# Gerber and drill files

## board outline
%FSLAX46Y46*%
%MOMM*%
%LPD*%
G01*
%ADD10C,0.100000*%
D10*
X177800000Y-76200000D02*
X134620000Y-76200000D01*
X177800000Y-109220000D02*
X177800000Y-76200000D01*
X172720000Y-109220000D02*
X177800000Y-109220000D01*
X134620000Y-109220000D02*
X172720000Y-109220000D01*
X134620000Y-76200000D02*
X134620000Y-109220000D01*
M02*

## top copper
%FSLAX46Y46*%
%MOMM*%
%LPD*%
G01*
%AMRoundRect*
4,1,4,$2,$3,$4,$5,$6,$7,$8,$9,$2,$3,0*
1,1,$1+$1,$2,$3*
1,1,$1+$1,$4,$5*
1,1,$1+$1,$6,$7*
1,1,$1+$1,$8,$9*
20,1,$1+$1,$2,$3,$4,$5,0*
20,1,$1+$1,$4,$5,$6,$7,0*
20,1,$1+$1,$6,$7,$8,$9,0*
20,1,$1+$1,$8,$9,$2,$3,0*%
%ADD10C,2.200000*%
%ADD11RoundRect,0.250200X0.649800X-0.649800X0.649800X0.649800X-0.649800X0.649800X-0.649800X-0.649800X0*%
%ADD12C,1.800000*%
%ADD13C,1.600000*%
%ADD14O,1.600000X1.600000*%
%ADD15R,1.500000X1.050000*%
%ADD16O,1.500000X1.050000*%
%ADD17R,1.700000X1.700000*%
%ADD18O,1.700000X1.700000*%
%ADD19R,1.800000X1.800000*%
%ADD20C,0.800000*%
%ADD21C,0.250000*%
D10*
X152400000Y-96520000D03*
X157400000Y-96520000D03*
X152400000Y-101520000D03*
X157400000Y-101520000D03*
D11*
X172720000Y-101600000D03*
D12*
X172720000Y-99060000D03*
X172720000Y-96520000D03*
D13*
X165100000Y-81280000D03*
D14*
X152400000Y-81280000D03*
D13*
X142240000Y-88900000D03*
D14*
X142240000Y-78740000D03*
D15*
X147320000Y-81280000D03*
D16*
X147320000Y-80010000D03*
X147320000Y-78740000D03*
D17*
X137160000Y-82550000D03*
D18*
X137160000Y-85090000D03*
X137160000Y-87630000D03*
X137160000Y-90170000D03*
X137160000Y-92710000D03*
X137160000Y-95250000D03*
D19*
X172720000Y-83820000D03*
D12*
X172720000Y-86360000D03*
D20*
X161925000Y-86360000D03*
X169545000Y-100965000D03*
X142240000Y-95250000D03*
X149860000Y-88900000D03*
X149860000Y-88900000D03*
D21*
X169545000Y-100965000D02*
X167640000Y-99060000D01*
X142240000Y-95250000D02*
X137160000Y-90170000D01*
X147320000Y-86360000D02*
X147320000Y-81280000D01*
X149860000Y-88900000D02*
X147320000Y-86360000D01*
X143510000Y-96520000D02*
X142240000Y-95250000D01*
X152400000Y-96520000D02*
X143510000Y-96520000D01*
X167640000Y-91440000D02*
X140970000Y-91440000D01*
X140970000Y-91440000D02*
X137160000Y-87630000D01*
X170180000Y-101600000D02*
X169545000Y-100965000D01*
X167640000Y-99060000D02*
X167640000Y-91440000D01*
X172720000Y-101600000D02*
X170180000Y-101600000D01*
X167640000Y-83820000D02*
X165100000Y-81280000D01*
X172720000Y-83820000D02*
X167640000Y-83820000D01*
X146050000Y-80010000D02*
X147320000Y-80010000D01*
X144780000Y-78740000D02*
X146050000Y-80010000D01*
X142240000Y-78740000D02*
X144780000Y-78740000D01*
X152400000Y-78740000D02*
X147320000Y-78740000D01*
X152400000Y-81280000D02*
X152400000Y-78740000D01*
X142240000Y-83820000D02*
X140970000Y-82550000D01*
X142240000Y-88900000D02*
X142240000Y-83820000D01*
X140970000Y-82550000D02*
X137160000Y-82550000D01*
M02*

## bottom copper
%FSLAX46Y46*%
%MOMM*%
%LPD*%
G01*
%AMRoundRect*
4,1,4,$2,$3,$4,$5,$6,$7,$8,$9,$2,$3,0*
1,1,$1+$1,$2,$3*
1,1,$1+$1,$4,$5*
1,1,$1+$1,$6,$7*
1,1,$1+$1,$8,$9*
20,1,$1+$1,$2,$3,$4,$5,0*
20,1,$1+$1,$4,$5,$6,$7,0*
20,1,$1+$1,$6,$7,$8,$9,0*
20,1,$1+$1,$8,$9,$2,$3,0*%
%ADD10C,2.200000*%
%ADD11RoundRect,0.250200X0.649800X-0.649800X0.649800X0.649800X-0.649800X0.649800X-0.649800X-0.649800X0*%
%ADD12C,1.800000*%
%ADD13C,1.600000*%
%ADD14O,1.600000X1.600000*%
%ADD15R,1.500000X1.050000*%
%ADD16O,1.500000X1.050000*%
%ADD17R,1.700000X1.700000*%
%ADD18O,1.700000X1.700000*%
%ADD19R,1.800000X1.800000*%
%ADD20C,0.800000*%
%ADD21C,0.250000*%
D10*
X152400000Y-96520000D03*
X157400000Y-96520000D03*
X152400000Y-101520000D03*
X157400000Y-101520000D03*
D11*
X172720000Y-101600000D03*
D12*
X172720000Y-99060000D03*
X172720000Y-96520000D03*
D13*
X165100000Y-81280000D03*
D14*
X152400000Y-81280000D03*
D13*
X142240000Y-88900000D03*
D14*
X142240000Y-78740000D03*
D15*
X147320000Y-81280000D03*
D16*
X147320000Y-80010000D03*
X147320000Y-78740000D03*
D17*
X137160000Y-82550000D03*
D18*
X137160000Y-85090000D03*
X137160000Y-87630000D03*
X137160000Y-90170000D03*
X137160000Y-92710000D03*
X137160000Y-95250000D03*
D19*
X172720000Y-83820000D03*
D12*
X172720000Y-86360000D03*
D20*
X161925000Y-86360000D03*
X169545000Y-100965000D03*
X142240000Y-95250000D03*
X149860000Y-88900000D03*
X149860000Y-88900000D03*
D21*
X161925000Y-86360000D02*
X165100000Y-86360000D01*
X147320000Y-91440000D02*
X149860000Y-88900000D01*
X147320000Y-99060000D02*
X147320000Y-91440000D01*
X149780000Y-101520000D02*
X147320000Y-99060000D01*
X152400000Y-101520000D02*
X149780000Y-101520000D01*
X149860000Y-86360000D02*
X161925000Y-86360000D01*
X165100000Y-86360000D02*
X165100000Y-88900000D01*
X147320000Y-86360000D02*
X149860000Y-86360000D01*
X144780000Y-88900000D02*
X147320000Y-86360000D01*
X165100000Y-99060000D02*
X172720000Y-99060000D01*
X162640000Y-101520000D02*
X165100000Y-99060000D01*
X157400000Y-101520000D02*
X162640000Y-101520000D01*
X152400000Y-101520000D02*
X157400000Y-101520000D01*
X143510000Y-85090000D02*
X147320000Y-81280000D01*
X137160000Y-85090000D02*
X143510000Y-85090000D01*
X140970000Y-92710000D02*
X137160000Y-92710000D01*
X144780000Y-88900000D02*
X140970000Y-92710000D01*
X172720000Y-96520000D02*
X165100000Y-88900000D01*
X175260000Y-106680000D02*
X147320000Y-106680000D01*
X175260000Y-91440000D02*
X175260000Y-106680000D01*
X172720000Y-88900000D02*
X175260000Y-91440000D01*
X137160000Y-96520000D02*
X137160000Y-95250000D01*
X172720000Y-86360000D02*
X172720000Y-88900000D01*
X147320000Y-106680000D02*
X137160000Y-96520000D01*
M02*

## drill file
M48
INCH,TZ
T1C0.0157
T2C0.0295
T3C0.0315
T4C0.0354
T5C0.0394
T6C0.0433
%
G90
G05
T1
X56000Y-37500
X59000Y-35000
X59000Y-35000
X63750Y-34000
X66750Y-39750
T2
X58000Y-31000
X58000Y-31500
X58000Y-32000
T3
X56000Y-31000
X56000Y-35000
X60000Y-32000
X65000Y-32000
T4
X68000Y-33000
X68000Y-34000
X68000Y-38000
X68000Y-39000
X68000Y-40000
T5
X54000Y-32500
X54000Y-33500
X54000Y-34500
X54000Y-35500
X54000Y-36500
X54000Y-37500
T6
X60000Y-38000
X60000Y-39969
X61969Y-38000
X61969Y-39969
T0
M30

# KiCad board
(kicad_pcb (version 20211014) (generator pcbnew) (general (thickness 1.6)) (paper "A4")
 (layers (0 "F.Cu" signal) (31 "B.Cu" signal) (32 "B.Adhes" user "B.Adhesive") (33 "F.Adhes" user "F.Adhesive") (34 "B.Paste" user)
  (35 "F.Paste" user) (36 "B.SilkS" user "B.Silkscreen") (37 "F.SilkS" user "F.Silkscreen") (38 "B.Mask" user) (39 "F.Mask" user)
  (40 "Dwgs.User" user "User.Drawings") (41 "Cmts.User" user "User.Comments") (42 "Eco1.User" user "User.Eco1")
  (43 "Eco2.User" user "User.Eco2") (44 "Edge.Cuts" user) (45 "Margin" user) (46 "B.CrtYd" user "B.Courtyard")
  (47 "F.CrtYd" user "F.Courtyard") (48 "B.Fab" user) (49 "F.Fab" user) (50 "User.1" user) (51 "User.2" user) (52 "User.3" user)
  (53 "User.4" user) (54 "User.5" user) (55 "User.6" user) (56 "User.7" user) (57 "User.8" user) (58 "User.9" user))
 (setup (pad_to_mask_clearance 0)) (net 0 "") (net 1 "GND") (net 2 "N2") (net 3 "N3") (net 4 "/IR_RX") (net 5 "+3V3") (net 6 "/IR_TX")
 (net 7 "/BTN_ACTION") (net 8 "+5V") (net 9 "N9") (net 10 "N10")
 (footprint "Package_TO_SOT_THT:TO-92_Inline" (layer "F.Cu") (at 147.32 81.28 90)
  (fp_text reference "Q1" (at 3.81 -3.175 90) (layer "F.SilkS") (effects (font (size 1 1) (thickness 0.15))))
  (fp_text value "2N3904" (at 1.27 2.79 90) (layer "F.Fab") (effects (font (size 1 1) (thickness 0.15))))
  (pad "1" thru_hole rect (at 0 0 90) (size 1.05 1.5) (drill 0.75) (layers *.Cu *.Mask) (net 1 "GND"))
  (pad "2" thru_hole oval (at 1.27 0 90) (size 1.05 1.5) (drill 0.75) (layers *.Cu *.Mask) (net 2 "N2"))
  (pad "3" thru_hole oval (at 2.54 0 90) (size 1.05 1.5) (drill 0.75) (layers *.Cu *.Mask) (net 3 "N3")))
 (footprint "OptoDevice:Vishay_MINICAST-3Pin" (layer "F.Cu") (at 172.72 101.6 90)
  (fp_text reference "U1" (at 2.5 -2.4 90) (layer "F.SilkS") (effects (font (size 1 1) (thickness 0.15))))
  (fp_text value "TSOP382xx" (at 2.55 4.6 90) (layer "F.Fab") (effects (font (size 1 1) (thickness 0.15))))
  (pad "1" thru_hole roundrect (at 0 0 90) (size 1.8 1.8) (drill 0.9) (layers *.Cu *.Mask) (roundrect_rratio 0.139) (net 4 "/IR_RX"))
  (pad "2" thru_hole circle (at 2.54 0 90) (size 1.8 1.8) (drill 0.9) (layers *.Cu *.Mask) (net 1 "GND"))
  (pad "3" thru_hole circle (at 5.08 0 90) (size 1.8 1.8) (drill 0.9) (layers *.Cu *.Mask) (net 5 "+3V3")))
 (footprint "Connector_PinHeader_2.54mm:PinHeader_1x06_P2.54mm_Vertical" (layer "F.Cu") (at 137.16 82.55)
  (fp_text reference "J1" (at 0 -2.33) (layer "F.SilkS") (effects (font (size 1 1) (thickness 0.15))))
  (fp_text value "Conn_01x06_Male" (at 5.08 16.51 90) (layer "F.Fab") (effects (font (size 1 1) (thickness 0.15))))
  (pad "1" thru_hole rect (at 0 0) (size 1.7 1.7) (drill 1) (layers *.Cu *.Mask) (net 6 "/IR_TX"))
  (pad "2" thru_hole oval (at 0 2.54) (size 1.7 1.7) (drill 1) (layers *.Cu *.Mask) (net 1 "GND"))
  (pad "3" thru_hole oval (at 0 5.08) (size 1.7 1.7) (drill 1) (layers *.Cu *.Mask) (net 4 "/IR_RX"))
  (pad "4" thru_hole oval (at 0 7.62) (size 1.7 1.7) (drill 1) (layers *.Cu *.Mask) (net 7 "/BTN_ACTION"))
  (pad "5" thru_hole oval (at 0 10.16) (size 1.7 1.7) (drill 1) (layers *.Cu *.Mask) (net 5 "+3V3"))
  (pad "6" thru_hole oval (at 0 12.7) (size 1.7 1.7) (drill 1) (layers *.Cu *.Mask) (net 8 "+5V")))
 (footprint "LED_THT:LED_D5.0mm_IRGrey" (layer "F.Cu") (at 172.72 83.82 -90)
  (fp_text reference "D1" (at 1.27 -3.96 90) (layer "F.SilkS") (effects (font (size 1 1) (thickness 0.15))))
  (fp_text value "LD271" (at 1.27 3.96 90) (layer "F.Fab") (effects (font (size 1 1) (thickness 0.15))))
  (pad "1" thru_hole rect (at 0 0 270) (size 1.8 1.8) (drill 0.9) (layers *.Cu *.Mask) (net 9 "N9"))
  (pad "2" thru_hole circle (at 2.54 0 270) (size 1.8 1.8) (drill 0.9) (layers *.Cu *.Mask) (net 8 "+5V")))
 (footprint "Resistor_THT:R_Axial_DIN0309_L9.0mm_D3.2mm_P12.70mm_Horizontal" (layer "F.Cu") (at 165.1 81.28 180)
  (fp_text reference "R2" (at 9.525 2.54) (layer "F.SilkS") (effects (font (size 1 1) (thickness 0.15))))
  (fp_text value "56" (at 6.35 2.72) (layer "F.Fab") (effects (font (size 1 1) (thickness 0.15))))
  (pad "1" thru_hole circle (at 0 0 180) (size 1.6 1.6) (drill 0.8) (layers *.Cu *.Mask) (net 9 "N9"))
  (pad "2" thru_hole oval (at 12.7 0 180) (size 1.6 1.6) (drill 0.8) (layers *.Cu *.Mask) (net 3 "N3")))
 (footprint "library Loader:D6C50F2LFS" (layer "F.Cu") (at 152.4 96.52)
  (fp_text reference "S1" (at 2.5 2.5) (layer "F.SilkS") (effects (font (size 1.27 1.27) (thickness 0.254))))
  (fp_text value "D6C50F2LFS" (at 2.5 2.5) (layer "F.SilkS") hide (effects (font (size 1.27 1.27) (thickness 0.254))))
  (pad "1" thru_hole circle locked (at 0 0) (size 2.2 2.2) (drill 1.1) (layers *.Cu *.Mask) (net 7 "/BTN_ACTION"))
  (pad "2" thru_hole circle locked (at 5 0) (size 2.2 2.2) (drill 1.1) (layers *.Cu *.Mask) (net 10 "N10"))
  (pad "3" thru_hole circle locked (at 0 5) (size 2.2 2.2) (drill 1.1) (layers *.Cu *.Mask) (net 1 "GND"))
  (pad "4" thru_hole circle locked (at 5 5) (size 2.2 2.2) (drill 1.1) (layers *.Cu *.Mask) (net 1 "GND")))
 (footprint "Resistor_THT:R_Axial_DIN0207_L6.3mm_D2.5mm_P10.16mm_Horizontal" (layer "F.Cu") (at 142.24 88.9 90)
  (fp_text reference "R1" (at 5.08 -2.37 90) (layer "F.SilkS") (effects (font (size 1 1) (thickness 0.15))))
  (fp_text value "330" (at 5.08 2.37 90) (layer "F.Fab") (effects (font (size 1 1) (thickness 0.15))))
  (pad "1" thru_hole circle (at 0 0 90) (size 1.6 1.6) (drill 0.8) (layers *.Cu *.Mask) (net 6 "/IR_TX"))
  (pad "2" thru_hole oval (at 10.16 0 90) (size 1.6 1.6) (drill 0.8) (layers *.Cu *.Mask) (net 2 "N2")))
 (gr_line (start 177.8 76.2) (end 134.62 76.2) (layer "Edge.Cuts") (width 0.1))
 (gr_line (start 134.62 109.22) (end 172.72 109.22) (layer "Edge.Cuts") (width 0.1))
 (gr_line (start 172.72 109.22) (end 177.8 109.22) (layer "Edge.Cuts") (width 0.1))
 (gr_line (start 177.8 109.22) (end 177.8 76.2) (layer "Edge.Cuts") (width 0.1))
 (gr_line (start 134.62 76.2) (end 134.62 109.22) (layer "Edge.Cuts") (width 0.1))
 (segment (start 172.72 83.82) (end 167.64 83.82) (width 0.25) (layer "F.Cu") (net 9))
 (segment (start 167.64 83.82) (end 165.1 81.28) (width 0.25) (layer "F.Cu") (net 9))
 (segment (start 147.32 106.68) (end 137.16 96.52) (width 0.25) (layer "B.Cu") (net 8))
 (segment (start 172.72 88.9) (end 175.26 91.44) (width 0.25) (layer "B.Cu") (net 8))
 (segment (start 175.26 91.44) (end 175.26 106.68) (width 0.25) (layer "B.Cu") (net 8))
 (segment (start 175.26 106.68) (end 147.32 106.68) (width 0.25) (layer "B.Cu") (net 8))
 (segment (start 137.16 96.52) (end 137.16 95.25) (width 0.25) (layer "B.Cu") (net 8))
 (segment (start 172.72 86.36) (end 172.72 88.9) (width 0.25) (layer "B.Cu") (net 8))
 (segment (start 142.24 88.9) (end 142.24 83.82) (width 0.25) (layer "F.Cu") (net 6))
 (segment (start 140.97 82.55) (end 137.16 82.55) (width 0.25) (layer "F.Cu") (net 6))
 (segment (start 142.24 83.82) (end 140.97 82.55) (width 0.25) (layer "F.Cu") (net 6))
 (segment (start 147.32 86.36) (end 147.32 81.28) (width 0.25) (layer "F.Cu") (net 1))
 (segment (start 149.86 88.9) (end 147.32 86.36) (width 0.25) (layer "F.Cu") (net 1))
 (via (at 149.86 88.9) (size 0.8) (drill 0.4) (layers "F.Cu" "B.Cu") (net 1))
 (via (at 149.86 88.9) (size 0.8) (drill 0.4) (layers "F.Cu" "B.Cu") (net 1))
 (segment (start 137.16 85.09) (end 143.51 85.09) (width 0.25) (layer "B.Cu") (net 1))
 (segment (start 152.4 101.52) (end 149.78 101.52) (width 0.25) (layer "B.Cu") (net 1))
 (segment (start 152.4 101.52) (end 157.4 101.52) (width 0.25) (layer "B.Cu") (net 1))
 (segment (start 143.51 85.09) (end 147.32 81.28) (width 0.25) (layer "B.Cu") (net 1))
 (segment (start 162.64 101.52) (end 165.1 99.06) (width 0.25) (layer "B.Cu") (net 1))
 (segment (start 157.4 101.52) (end 162.64 101.52) (width 0.25) (layer "B.Cu") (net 1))
 (segment (start 147.32 91.44) (end 149.86 88.9) (width 0.25) (layer "B.Cu") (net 1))
 (segment (start 149.78 101.52) (end 147.32 99.06) (width 0.25) (layer "B.Cu") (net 1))
 (segment (start 147.32 99.06) (end 147.32 91.44) (width 0.25) (layer "B.Cu") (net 1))
 (segment (start 165.1 99.06) (end 172.72 99.06) (width 0.25) (layer "B.Cu") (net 1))
 (segment (start 172.72 101.6) (end 170.18 101.6) (width 0.25) (layer "F.Cu") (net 4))
 (segment (start 170.18 101.6) (end 169.545 100.965) (width 0.25) (layer "F.Cu") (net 4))
 (segment (start 140.97 91.44) (end 137.16 87.63) (width 0.25) (layer "F.Cu") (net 4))
 (segment (start 167.64 91.44) (end 140.97 91.44) (width 0.25) (layer "F.Cu") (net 4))
 (segment (start 167.64 99.06) (end 167.64 91.44) (width 0.25) (layer "F.Cu") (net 4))
 (segment (start 169.545 100.965) (end 167.64 99.06) (width 0.25) (layer "F.Cu") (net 4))
 (via (at 169.545 100.965) (size 0.8) (drill 0.4) (layers "F.Cu" "B.Cu") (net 4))
 (segment (start 152.4 96.52) (end 143.51 96.52) (width 0.25) (layer "F.Cu") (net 7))
 (segment (start 142.24 95.25) (end 137.16 90.17) (width 0.25) (layer "F.Cu") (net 7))
 (segment (start 143.51 96.52) (end 142.24 95.25) (width 0.25) (layer "F.Cu") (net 7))
 (via (at 142.24 95.25) (size 0.8) (drill 0.4) (layers "F.Cu" "B.Cu") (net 7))
 (via (at 161.925 86.36) (size 0.8) (drill 0.4) (layers "F.Cu" "B.Cu") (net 5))
 (segment (start 144.78 88.9) (end 140.97 92.71) (width 0.25) (layer "B.Cu") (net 5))
 (segment (start 147.32 86.36) (end 149.86 86.36) (width 0.25) (layer "B.Cu") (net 5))
 (segment (start 149.86 86.36) (end 161.925 86.36) (width 0.25) (layer "B.Cu") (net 5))
 (segment (start 140.97 92.71) (end 137.16 92.71) (width 0.25) (layer "B.Cu") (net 5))
 (segment (start 161.925 86.36) (end 165.1 86.36) (width 0.25) (layer "B.Cu") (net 5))
 (segment (start 144.78 88.9) (end 147.32 86.36) (width 0.25) (layer "B.Cu") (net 5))
 (segment (start 165.1 86.36) (end 165.1 88.9) (width 0.25) (layer "B.Cu") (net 5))
 (segment (start 172.72 96.52) (end 165.1 88.9) (width 0.25) (layer "B.Cu") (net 5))
 (segment (start 142.24 78.74) (end 144.78 78.74) (width 0.25) (layer "F.Cu") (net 2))
 (segment (start 144.78 78.74) (end 146.05 80.01) (width 0.25) (layer "F.Cu") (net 2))
 (segment (start 146.05 80.01) (end 147.32 80.01) (width 0.25) (layer "F.Cu") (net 2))
 (segment (start 152.4 81.28) (end 152.4 78.74) (width 0.25) (layer "F.Cu") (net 3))
 (segment (start 152.4 78.74) (end 147.32 78.74) (width 0.25) (layer "F.Cu") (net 3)))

